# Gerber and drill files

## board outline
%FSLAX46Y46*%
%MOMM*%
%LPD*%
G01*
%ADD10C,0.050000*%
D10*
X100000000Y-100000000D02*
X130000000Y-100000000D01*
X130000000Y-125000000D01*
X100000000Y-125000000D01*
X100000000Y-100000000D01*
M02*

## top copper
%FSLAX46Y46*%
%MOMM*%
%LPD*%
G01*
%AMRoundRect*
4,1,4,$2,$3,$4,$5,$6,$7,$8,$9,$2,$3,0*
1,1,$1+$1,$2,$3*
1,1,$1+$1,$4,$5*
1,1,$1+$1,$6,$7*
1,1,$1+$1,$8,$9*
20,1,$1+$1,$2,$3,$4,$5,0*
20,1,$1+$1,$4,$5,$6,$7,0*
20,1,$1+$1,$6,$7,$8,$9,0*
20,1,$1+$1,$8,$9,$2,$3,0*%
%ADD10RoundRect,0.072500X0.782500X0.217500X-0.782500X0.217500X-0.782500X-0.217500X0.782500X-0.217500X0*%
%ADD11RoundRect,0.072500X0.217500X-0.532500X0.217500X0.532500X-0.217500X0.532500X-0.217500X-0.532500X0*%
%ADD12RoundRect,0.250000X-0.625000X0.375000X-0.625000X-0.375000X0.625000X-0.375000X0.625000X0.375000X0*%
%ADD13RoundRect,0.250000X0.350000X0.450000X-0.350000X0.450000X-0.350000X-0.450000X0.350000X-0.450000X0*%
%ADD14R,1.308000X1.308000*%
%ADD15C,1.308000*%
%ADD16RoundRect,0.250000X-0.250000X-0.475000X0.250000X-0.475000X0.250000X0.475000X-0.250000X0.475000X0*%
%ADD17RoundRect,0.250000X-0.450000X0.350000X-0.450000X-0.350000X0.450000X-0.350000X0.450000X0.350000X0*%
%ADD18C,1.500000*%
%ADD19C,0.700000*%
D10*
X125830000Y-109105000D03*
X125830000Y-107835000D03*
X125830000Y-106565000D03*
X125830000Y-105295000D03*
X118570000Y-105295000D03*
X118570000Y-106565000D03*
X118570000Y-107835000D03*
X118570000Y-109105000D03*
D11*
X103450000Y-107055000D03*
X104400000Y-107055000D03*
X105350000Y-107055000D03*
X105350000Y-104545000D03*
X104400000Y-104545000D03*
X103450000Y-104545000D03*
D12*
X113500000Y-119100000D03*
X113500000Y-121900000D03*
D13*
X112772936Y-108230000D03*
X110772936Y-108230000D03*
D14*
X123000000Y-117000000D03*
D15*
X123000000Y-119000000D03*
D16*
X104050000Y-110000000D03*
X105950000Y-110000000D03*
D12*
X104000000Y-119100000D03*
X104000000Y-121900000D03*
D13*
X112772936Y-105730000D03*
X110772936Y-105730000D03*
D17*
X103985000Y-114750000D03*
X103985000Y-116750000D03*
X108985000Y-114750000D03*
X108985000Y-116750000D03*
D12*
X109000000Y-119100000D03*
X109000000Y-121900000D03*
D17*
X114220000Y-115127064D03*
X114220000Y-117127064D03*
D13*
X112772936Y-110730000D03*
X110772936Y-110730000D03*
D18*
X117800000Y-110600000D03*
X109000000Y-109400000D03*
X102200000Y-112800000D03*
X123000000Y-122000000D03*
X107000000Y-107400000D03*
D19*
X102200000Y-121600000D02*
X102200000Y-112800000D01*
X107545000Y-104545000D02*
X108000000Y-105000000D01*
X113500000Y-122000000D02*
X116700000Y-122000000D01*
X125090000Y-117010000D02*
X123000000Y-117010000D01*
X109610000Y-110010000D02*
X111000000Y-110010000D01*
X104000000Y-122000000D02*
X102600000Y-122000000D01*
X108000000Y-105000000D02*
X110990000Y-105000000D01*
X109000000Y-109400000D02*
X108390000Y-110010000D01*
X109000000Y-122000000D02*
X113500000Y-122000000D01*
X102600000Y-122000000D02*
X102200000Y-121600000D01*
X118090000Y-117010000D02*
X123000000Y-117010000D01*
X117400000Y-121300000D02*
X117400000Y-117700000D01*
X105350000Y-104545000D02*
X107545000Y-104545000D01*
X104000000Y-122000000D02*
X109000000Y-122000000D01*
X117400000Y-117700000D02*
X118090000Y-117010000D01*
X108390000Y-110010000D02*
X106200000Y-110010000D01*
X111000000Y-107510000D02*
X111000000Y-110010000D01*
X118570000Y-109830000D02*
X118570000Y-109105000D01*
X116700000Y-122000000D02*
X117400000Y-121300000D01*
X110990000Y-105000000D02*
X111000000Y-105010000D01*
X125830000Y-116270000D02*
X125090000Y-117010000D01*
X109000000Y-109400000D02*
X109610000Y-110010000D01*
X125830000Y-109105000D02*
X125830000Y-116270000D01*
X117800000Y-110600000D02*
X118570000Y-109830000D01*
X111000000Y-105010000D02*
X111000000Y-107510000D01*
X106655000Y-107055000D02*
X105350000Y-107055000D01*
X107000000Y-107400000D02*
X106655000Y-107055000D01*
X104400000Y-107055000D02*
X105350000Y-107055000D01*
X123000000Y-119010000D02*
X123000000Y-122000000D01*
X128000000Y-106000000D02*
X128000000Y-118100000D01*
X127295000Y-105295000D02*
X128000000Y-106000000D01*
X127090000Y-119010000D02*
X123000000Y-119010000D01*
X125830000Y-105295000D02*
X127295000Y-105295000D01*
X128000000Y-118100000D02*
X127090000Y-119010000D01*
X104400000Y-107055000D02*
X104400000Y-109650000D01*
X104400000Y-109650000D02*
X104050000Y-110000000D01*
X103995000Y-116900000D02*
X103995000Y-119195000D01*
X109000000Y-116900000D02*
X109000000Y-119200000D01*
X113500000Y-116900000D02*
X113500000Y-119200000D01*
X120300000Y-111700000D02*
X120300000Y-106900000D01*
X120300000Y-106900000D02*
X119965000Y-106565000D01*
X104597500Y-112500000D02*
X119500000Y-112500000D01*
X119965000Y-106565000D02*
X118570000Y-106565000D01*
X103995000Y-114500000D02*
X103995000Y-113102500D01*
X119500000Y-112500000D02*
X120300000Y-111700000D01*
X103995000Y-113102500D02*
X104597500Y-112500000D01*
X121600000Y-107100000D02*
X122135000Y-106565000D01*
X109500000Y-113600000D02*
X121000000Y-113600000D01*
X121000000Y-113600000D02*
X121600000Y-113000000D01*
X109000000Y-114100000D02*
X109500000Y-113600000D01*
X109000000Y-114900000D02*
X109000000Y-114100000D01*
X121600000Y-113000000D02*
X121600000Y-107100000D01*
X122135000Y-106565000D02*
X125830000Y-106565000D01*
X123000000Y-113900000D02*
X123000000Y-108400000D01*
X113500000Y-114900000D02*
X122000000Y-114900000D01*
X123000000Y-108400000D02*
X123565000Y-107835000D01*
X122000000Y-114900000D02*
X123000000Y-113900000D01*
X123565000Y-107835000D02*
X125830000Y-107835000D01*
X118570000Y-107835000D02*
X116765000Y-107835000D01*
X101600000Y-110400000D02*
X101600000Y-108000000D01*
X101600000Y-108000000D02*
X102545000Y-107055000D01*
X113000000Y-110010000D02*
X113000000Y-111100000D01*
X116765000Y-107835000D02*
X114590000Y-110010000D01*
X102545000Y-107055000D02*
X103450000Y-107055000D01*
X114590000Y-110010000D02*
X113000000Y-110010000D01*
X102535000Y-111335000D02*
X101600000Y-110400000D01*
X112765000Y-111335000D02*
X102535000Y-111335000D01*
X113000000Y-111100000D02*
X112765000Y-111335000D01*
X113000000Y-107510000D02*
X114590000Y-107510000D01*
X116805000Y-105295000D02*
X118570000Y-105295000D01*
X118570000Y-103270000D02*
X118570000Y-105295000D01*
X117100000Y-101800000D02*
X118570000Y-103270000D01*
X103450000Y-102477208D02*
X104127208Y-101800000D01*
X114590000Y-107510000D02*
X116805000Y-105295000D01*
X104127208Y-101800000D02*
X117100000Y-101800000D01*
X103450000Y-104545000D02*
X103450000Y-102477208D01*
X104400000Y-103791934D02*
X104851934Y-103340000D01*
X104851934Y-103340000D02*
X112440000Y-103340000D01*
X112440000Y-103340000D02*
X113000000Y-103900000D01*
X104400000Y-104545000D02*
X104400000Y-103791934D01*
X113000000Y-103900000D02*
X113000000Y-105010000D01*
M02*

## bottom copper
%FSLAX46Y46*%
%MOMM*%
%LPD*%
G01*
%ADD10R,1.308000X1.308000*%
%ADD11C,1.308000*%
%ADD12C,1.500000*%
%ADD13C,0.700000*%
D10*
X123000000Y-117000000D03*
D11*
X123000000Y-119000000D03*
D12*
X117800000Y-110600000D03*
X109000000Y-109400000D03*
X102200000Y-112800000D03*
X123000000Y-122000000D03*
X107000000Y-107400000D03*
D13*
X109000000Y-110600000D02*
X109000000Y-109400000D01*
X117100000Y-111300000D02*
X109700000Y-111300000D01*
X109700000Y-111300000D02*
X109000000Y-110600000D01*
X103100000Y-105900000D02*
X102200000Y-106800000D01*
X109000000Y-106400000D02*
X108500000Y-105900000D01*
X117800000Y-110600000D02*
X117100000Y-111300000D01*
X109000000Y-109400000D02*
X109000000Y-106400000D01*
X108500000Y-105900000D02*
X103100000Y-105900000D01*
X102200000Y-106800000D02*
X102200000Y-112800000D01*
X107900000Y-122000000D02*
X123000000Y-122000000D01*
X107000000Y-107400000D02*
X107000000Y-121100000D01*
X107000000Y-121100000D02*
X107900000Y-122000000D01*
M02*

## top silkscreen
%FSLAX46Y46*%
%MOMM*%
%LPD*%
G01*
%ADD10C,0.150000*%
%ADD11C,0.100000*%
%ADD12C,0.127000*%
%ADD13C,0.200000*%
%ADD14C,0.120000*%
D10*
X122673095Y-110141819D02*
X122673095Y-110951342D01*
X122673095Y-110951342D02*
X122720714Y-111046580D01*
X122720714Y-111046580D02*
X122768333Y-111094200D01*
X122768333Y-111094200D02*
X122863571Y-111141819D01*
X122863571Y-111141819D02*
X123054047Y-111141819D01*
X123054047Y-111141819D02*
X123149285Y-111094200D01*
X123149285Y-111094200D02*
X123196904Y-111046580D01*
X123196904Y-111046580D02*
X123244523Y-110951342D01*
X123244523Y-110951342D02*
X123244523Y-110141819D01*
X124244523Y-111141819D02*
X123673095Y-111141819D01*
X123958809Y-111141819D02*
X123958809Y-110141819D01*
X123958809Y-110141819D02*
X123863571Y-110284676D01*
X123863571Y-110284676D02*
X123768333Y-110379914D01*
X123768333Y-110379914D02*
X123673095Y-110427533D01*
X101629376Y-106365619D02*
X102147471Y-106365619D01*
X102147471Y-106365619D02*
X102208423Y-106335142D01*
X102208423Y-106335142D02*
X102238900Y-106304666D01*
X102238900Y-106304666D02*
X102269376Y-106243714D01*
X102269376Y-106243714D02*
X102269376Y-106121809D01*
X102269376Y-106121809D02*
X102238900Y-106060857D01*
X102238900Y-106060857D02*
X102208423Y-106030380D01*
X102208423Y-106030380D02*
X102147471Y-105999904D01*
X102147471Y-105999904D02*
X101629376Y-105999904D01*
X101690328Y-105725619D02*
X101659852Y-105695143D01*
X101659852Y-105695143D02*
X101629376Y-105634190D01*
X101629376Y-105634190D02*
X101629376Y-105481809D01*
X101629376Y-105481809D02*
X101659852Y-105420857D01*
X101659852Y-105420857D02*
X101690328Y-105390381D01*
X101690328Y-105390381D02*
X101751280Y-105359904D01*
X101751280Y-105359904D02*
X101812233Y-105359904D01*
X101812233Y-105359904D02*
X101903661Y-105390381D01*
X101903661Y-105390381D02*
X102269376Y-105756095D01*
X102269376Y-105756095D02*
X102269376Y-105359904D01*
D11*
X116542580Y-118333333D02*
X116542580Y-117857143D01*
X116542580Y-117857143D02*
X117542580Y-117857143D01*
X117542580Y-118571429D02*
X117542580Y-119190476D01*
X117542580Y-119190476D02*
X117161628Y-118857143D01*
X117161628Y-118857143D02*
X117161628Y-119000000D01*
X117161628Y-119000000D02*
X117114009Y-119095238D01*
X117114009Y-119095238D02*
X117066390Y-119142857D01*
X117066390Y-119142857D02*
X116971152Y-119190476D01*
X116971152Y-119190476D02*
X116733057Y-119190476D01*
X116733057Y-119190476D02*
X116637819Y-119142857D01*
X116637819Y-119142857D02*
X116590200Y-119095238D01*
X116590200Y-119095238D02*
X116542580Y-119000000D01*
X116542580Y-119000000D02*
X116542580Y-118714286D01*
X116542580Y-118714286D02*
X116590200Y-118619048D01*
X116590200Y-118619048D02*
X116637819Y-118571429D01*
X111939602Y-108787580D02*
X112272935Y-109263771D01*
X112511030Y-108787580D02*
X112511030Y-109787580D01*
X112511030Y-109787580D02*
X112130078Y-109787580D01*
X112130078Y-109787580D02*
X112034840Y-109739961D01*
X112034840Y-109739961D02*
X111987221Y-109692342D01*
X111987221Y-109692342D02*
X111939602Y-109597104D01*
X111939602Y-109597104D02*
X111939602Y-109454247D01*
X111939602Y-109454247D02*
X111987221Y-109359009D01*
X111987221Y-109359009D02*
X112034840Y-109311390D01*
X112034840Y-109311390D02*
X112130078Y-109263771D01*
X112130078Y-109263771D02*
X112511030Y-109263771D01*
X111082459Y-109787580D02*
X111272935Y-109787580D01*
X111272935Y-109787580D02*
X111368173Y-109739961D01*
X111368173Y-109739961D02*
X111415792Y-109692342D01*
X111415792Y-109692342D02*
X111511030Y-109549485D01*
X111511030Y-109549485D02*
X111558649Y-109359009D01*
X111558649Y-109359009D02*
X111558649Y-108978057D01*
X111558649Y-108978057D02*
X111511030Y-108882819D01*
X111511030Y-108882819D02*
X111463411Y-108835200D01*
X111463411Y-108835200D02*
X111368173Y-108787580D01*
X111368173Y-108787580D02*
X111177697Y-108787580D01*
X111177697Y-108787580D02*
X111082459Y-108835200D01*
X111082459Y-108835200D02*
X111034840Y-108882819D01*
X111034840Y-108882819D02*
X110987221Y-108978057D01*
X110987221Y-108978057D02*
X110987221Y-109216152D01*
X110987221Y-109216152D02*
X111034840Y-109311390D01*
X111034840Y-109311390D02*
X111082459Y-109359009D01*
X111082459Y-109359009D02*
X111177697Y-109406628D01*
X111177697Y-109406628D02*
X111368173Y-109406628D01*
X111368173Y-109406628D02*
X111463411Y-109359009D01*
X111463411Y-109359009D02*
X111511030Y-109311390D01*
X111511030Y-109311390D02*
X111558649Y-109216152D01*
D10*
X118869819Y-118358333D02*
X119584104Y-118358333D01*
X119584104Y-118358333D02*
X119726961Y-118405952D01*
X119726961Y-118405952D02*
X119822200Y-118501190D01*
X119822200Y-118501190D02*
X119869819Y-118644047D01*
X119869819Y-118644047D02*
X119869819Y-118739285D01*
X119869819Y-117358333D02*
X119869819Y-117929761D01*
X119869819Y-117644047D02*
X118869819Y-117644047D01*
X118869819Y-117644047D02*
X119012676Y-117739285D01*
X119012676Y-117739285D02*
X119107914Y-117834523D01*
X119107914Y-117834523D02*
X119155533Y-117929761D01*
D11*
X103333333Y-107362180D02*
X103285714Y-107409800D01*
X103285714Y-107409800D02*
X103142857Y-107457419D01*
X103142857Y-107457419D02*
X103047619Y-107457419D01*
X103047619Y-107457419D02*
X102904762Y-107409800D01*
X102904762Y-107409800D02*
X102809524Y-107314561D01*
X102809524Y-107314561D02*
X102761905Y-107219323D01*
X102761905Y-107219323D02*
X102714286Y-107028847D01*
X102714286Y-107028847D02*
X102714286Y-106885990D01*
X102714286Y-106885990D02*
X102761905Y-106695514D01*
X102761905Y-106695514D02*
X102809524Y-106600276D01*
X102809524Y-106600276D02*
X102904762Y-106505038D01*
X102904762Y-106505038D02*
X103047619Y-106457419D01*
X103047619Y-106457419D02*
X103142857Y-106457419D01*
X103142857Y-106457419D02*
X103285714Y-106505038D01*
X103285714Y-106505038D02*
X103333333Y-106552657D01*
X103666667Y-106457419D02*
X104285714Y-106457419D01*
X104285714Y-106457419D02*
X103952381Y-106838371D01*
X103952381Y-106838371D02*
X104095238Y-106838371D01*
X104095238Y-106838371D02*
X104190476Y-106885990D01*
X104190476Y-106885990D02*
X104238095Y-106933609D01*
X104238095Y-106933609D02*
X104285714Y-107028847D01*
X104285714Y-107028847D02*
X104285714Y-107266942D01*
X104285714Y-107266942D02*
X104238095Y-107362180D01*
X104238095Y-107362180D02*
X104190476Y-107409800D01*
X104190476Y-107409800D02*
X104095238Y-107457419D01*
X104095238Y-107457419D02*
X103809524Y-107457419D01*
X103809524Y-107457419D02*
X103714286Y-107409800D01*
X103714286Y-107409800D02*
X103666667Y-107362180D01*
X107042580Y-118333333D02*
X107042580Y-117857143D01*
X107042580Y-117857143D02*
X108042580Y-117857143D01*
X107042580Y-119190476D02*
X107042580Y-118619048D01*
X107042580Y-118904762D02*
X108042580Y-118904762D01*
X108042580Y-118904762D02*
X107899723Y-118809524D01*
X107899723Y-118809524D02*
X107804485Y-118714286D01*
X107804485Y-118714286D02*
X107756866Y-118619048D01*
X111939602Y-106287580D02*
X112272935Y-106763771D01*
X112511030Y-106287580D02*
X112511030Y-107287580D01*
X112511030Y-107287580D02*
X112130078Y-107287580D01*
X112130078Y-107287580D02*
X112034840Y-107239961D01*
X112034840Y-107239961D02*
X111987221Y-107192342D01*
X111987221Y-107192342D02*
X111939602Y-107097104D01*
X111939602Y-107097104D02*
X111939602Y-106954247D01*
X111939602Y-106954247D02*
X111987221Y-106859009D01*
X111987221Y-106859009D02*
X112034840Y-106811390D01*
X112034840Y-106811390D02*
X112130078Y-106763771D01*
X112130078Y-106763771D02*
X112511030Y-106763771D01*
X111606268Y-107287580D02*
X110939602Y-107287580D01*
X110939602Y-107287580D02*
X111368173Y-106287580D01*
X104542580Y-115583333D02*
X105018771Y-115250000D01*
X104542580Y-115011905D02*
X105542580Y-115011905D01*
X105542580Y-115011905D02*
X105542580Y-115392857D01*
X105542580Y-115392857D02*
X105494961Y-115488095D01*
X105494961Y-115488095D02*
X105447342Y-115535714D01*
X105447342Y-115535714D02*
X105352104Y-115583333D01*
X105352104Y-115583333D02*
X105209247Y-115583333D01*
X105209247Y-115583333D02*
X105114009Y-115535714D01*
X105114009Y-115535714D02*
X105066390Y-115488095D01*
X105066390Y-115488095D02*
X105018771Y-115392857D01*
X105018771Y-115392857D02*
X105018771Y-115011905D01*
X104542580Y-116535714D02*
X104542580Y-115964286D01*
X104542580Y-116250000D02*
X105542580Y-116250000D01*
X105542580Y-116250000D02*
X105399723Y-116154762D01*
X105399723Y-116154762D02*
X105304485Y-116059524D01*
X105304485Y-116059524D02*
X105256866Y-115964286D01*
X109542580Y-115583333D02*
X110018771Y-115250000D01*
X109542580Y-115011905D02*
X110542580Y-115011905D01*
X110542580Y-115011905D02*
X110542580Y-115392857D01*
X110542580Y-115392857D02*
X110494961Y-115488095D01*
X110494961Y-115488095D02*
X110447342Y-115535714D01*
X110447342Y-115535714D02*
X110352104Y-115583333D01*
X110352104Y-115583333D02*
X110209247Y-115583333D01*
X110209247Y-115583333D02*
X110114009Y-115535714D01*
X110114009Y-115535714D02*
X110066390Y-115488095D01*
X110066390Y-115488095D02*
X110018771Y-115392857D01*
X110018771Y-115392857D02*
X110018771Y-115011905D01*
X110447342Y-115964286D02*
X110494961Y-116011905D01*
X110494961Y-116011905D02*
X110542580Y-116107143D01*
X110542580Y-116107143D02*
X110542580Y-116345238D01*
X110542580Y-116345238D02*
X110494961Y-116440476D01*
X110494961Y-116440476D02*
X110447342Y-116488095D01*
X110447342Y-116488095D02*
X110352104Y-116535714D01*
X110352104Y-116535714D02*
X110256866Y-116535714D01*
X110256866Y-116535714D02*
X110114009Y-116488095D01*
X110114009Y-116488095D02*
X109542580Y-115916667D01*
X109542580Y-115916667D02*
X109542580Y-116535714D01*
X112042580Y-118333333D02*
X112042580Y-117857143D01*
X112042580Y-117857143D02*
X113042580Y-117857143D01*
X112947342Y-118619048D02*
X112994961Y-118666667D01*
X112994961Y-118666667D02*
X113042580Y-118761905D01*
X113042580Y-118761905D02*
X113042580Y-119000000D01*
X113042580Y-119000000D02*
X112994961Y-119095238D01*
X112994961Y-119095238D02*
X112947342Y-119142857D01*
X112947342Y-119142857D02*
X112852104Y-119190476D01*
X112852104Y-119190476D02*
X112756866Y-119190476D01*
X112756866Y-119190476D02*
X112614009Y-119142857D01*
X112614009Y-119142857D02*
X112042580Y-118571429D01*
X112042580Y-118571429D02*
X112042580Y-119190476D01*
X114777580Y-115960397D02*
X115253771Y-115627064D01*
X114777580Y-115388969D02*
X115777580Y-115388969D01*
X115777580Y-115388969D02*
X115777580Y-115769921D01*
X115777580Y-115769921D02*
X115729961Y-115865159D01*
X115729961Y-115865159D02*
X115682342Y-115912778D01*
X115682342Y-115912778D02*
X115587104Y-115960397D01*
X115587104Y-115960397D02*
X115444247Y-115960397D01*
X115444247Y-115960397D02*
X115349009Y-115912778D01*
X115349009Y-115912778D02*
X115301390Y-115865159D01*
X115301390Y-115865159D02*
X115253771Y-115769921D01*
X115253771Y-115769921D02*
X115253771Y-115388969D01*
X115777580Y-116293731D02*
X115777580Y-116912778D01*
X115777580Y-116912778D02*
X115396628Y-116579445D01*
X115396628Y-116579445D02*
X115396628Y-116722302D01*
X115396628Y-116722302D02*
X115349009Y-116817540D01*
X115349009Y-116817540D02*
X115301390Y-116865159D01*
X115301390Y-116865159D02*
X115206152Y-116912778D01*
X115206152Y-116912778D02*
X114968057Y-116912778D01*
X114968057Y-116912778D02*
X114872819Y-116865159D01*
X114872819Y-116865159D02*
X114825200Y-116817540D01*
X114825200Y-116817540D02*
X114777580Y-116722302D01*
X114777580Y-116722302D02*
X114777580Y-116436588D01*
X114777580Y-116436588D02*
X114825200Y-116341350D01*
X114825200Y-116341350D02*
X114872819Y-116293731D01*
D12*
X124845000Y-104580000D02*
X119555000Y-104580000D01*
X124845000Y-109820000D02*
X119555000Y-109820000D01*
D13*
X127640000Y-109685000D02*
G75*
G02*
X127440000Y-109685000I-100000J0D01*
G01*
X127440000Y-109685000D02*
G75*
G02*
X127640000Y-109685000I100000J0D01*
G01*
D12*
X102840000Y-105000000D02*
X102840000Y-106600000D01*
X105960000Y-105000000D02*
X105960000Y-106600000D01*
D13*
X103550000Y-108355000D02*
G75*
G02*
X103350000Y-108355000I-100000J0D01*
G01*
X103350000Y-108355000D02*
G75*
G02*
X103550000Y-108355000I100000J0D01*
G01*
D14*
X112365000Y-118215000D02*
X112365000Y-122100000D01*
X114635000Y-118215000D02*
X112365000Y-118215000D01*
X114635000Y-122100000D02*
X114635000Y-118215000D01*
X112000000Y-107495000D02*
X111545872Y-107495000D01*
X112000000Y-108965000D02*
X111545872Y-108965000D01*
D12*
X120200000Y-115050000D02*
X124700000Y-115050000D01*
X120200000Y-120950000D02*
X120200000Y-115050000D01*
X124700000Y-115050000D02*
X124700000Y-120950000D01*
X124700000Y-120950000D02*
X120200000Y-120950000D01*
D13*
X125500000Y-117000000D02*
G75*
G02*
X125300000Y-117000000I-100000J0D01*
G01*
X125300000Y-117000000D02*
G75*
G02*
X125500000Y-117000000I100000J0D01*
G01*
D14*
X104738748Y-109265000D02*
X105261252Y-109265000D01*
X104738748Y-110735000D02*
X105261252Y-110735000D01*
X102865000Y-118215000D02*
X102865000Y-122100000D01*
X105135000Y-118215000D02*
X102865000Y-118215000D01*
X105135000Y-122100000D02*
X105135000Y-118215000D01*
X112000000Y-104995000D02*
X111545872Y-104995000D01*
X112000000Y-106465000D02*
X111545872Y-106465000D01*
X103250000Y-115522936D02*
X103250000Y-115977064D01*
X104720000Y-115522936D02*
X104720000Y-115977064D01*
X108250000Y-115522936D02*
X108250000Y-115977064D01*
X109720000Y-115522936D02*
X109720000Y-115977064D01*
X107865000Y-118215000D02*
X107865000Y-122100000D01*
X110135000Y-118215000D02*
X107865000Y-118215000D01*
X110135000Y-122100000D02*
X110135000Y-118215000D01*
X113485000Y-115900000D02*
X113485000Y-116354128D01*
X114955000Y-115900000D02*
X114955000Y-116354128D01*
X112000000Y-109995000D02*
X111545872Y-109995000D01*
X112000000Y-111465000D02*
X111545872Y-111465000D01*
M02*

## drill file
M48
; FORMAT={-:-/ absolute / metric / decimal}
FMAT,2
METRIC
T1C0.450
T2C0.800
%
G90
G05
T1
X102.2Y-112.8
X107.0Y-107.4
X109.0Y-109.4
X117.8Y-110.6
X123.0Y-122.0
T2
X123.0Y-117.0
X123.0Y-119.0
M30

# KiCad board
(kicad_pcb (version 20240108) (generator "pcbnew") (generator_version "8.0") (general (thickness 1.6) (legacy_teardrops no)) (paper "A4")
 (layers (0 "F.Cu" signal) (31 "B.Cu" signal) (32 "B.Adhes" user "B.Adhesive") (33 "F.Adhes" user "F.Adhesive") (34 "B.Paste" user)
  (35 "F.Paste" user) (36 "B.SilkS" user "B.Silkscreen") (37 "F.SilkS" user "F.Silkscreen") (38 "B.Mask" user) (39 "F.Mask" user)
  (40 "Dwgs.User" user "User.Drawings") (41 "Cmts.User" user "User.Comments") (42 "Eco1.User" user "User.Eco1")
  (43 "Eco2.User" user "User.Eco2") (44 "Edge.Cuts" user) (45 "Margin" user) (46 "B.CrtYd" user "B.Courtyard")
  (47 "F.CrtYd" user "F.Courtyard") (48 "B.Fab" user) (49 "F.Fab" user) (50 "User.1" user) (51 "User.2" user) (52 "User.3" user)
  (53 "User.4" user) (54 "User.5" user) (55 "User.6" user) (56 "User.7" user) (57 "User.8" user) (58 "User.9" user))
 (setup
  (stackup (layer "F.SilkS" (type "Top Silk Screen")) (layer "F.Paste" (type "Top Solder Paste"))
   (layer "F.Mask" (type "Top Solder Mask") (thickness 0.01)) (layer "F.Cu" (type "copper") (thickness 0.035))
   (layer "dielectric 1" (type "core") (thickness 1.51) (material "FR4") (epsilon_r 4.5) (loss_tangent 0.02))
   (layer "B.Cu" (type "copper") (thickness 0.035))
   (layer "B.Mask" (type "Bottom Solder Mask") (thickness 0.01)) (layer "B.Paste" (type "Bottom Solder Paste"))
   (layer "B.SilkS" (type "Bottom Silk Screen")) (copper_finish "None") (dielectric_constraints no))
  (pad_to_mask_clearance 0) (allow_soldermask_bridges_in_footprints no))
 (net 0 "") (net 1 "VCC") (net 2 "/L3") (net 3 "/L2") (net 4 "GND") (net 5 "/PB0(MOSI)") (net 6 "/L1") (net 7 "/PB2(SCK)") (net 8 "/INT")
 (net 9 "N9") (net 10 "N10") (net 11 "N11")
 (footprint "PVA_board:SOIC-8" (layer "F.Cu") (at 122.2 107.2 180)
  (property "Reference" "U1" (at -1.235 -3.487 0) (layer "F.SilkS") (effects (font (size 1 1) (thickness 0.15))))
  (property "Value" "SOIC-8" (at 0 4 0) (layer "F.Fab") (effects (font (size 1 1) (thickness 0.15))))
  (fp_line (start -2.645 2.62) (end 2.645 2.62) (stroke (width 0.127) (type solid)) (layer "F.SilkS"))
  (fp_line (start -2.645 -2.62) (end 2.645 -2.62) (stroke (width 0.127) (type solid)) (layer "F.SilkS"))
  (fp_circle (center -5.34 -2.485) (end -5.24 -2.485) (stroke (width 0.2) (type solid)) (fill none) (layer "F.SilkS"))
  (pad "1" smd roundrect (at -3.63 -1.905 180) (size 1.71 0.58) (layers "F.Cu" "F.Paste" "F.Mask") (roundrect_rratio 0.125) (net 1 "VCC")
   (solder_mask_margin 0.102))
  (pad "2" smd roundrect (at -3.63 -0.635 180) (size 1.71 0.58) (layers "F.Cu" "F.Paste" "F.Mask") (roundrect_rratio 0.125) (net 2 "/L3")
   (solder_mask_margin 0.102))
  (pad "3" smd roundrect (at -3.63 0.635 180) (size 1.71 0.58) (layers "F.Cu" "F.Paste" "F.Mask") (roundrect_rratio 0.125) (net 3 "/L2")
   (solder_mask_margin 0.102))
  (pad "4" smd roundrect (at -3.63 1.905 180) (size 1.71 0.58) (layers "F.Cu" "F.Paste" "F.Mask") (roundrect_rratio 0.125) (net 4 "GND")
   (solder_mask_margin 0.102))
  (pad "5" smd roundrect (at 3.63 1.905 180) (size 1.71 0.58) (layers "F.Cu" "F.Paste" "F.Mask") (roundrect_rratio 0.125)
   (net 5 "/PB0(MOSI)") (solder_mask_margin 0.102))
  (pad "6" smd roundrect (at 3.63 0.635 180) (size 1.71 0.58) (layers "F.Cu" "F.Paste" "F.Mask") (roundrect_rratio 0.125) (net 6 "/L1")
   (solder_mask_margin 0.102))
  (pad "7" smd roundrect (at 3.63 -0.635 180) (size 1.71 0.58) (layers "F.Cu" "F.Paste" "F.Mask") (roundrect_rratio 0.125)
   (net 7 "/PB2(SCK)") (solder_mask_margin 0.102))
  (pad "8" smd roundrect (at 3.63 -1.905 180) (size 1.71 0.58) (layers "F.Cu" "F.Paste" "F.Mask") (roundrect_rratio 0.125) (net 1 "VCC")
   (solder_mask_margin 0.102)))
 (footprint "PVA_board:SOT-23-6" (layer "F.Cu") (at 104.4 105.8 90)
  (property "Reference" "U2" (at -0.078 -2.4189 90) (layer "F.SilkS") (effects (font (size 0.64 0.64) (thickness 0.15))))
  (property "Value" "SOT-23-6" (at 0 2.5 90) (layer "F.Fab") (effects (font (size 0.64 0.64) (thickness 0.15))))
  (fp_line (start 0.8 -1.56) (end -0.8 -1.56) (stroke (width 0.127) (type solid)) (layer "F.SilkS"))
  (fp_line (start 0.8 1.56) (end -0.8 1.56) (stroke (width 0.127) (type solid)) (layer "F.SilkS"))
  (fp_circle (center -2.555 -0.95) (end -2.455 -0.95) (stroke (width 0.2) (type solid)) (fill none) (layer "F.SilkS"))
  (pad "1" smd roundrect (at -1.255 -0.95 90) (size 1.21 0.58) (layers "F.Cu" "F.Paste" "F.Mask") (roundrect_rratio 0.125)
   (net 7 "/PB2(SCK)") (solder_mask_margin 0.102))
  (pad "2" smd roundrect (at -1.255 0 90) (size 1.21 0.58) (layers "F.Cu" "F.Paste" "F.Mask") (roundrect_rratio 0.125) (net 4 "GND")
   (solder_mask_margin 0.102))
  (pad "3" smd roundrect (at -1.255 0.95 90) (size 1.21 0.58) (layers "F.Cu" "F.Paste" "F.Mask") (roundrect_rratio 0.125) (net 4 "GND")
   (solder_mask_margin 0.102))
  (pad "4" smd roundrect (at 1.255 0.95 90) (size 1.21 0.58) (layers "F.Cu" "F.Paste" "F.Mask") (roundrect_rratio 0.125) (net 1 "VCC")
   (solder_mask_margin 0.102))
  (pad "5" smd roundrect (at 1.255 0 90) (size 1.21 0.58) (layers "F.Cu" "F.Paste" "F.Mask") (roundrect_rratio 0.125) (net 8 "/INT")
   (solder_mask_margin 0.102))
  (pad "6" smd roundrect (at 1.255 -0.95 90) (size 1.21 0.58) (layers "F.Cu" "F.Paste" "F.Mask") (roundrect_rratio 0.125)
   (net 5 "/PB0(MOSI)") (solder_mask_margin 0.102)))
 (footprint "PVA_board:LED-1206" (layer "F.Cu") (at 113.5 120.5 -90)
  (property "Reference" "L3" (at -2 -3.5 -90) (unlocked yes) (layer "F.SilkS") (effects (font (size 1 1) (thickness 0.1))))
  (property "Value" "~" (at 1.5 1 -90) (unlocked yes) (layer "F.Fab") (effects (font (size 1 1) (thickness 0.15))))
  (fp_line (start -2.285 1.135) (end 1.6 1.135) (stroke (width 0.12) (type solid)) (layer "F.SilkS"))
  (fp_line (start -2.285 -1.135) (end -2.285 1.135) (stroke (width 0.12) (type solid)) (layer "F.SilkS"))
  (fp_line (start 1.6 -1.135) (end -2.285 -1.135) (stroke (width 0.12) (type solid)) (layer "F.SilkS"))
  (pad "1" smd roundrect (at -1.4 0 270) (size 1.25 1.75) (layers "F.Cu" "F.Paste" "F.Mask") (roundrect_rratio 0.2) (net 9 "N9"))
  (pad "2" smd roundrect (at 1.4 0 270) (size 1.25 1.75) (layers "F.Cu" "F.Paste" "F.Mask") (roundrect_rratio 0.2) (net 1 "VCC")))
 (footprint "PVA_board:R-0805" (layer "F.Cu") (at 111.772936 108.245 180)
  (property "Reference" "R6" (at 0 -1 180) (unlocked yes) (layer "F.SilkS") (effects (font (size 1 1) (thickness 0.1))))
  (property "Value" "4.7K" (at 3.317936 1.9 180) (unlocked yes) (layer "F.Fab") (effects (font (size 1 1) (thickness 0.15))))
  (fp_line (start -0.227064 0.75) (end 0.227064 0.75) (stroke (width 0.12) (type solid)) (layer "F.SilkS"))
  (fp_line (start -0.227064 -0.72) (end 0.227064 -0.72) (stroke (width 0.12) (type solid)) (layer "F.SilkS"))
  (pad "1" smd roundrect (at -1 0.015 180) (size 1.2 1.4) (layers "F.Cu" "F.Paste" "F.Mask") (roundrect_rratio 0.208333)
   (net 5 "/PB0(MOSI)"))
  (pad "2" smd roundrect (at 1 0.015 180) (size 1.2 1.4) (layers "F.Cu" "F.Paste" "F.Mask") (roundrect_rratio 0.208333) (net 1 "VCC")))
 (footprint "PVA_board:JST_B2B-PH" (layer "F.Cu") (at 123 118 90)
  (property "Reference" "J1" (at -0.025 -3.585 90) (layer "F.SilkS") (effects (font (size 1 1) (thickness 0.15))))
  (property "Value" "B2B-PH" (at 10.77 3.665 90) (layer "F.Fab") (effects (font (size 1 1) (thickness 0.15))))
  (fp_line (start 2.95 -2.8) (end 2.95 1.7) (stroke (width 0.127) (type solid)) (layer "F.SilkS"))
  (fp_line (start -2.95 -2.8) (end 2.95 -2.8) (stroke (width 0.127) (type solid)) (layer "F.SilkS"))
  (fp_line (start 2.95 1.7) (end -2.95 1.7) (stroke (width 0.127) (type solid)) (layer "F.SilkS"))
  (fp_line (start -2.95 1.7) (end -2.95 -2.8) (stroke (width 0.127) (type solid)) (layer "F.SilkS"))
  (fp_circle (center 1 2.4) (end 1.1 2.4) (stroke (width 0.2) (type solid)) (fill none) (layer "F.SilkS"))
  (pad "1" thru_hole rect (at 1 0 90) (size 1.308 1.308) (drill 0.8) (layers "*.Cu" "*.Mask") (remove_unused_layers no) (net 1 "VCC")
   (solder_mask_margin 0.102))
  (pad "2" thru_hole circle (at -1 0 90) (size 1.308 1.308) (drill 0.8) (layers "*.Cu" "*.Mask") (remove_unused_layers no) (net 4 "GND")
   (solder_mask_margin 0.102)))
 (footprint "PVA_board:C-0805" (layer "F.Cu") (at 105 110)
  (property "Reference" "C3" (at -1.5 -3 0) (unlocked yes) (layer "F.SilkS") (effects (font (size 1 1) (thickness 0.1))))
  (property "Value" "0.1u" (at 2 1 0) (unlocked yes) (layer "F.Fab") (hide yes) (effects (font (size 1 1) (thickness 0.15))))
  (fp_line (start -0.261252 -0.735) (end 0.261252 -0.735) (stroke (width 0.12) (type solid)) (layer "F.SilkS"))
  (fp_line (start -0.261252 0.735) (end 0.261252 0.735) (stroke (width 0.12) (type solid)) (layer "F.SilkS"))
  (pad "1" smd roundrect (at -0.95 0) (size 1 1.45) (layers "F.Cu" "F.Paste" "F.Mask") (roundrect_rratio 0.25) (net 4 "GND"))
  (pad "2" smd roundrect (at 0.95 0) (size 1 1.45) (layers "F.Cu" "F.Paste" "F.Mask") (roundrect_rratio 0.25) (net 1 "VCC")))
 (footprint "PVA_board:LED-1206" (layer "F.Cu") (at 104 120.5 -90)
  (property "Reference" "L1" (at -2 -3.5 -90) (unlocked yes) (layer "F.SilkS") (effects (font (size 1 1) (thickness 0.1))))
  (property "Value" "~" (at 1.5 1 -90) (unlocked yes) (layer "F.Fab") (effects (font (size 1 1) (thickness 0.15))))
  (fp_line (start -2.285 1.135) (end 1.6 1.135) (stroke (width 0.12) (type solid)) (layer "F.SilkS"))
  (fp_line (start -2.285 -1.135) (end -2.285 1.135) (stroke (width 0.12) (type solid)) (layer "F.SilkS"))
  (fp_line (start 1.6 -1.135) (end -2.285 -1.135) (stroke (width 0.12) (type solid)) (layer "F.SilkS"))
  (pad "1" smd roundrect (at -1.4 0 270) (size 1.25 1.75) (layers "F.Cu" "F.Paste" "F.Mask") (roundrect_rratio 0.2) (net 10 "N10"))
  (pad "2" smd roundrect (at 1.4 0 270) (size 1.25 1.75) (layers "F.Cu" "F.Paste" "F.Mask") (roundrect_rratio 0.2) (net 1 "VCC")))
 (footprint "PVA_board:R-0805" (layer "F.Cu") (at 111.772936 105.745 180)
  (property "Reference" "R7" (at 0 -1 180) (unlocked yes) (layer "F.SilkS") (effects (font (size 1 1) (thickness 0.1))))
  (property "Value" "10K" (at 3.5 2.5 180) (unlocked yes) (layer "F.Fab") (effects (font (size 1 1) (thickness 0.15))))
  (fp_line (start -0.227064 0.75) (end 0.227064 0.75) (stroke (width 0.12) (type solid)) (layer "F.SilkS"))
  (fp_line (start -0.227064 -0.72) (end 0.227064 -0.72) (stroke (width 0.12) (type solid)) (layer "F.SilkS"))
  (pad "1" smd roundrect (at -1 0.015 180) (size 1.2 1.4) (layers "F.Cu" "F.Paste" "F.Mask") (roundrect_rratio 0.208333) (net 8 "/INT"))
  (pad "2" smd roundrect (at 1 0.015 180) (size 1.2 1.4) (layers "F.Cu" "F.Paste" "F.Mask") (roundrect_rratio 0.208333) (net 1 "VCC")))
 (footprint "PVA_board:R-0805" (layer "F.Cu") (at 104 115.75 -90)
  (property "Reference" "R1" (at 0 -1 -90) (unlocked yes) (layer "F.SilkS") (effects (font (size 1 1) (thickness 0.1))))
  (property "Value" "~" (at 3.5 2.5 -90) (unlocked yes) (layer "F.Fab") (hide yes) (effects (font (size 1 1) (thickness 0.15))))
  (fp_line (start -0.227064 0.75) (end 0.227064 0.75) (stroke (width 0.12) (type solid)) (layer "F.SilkS"))
  (fp_line (start -0.227064 -0.72) (end 0.227064 -0.72) (stroke (width 0.12) (type solid)) (layer "F.SilkS"))
  (pad "1" smd roundrect (at -1 0.015 270) (size 1.2 1.4) (layers "F.Cu" "F.Paste" "F.Mask") (roundrect_rratio 0.208333) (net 6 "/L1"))
  (pad "2" smd roundrect (at 1 0.015 270) (size 1.2 1.4) (layers "F.Cu" "F.Paste" "F.Mask") (roundrect_rratio 0.208333) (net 10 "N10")))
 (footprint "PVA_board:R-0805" (layer "F.Cu") (at 109 115.75 -90)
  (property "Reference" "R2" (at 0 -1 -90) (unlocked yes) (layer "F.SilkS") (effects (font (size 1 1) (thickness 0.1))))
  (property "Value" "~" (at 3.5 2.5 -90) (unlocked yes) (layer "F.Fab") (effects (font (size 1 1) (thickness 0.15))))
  (fp_line (start -0.227064 0.75) (end 0.227064 0.75) (stroke (width 0.12) (type solid)) (layer "F.SilkS"))
  (fp_line (start -0.227064 -0.72) (end 0.227064 -0.72) (stroke (width 0.12) (type solid)) (layer "F.SilkS"))
  (pad "1" smd roundrect (at -1 0.015 270) (size 1.2 1.4) (layers "F.Cu" "F.Paste" "F.Mask") (roundrect_rratio 0.208333) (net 3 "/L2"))
  (pad "2" smd roundrect (at 1 0.015 270) (size 1.2 1.4) (layers "F.Cu" "F.Paste" "F.Mask") (roundrect_rratio 0.208333) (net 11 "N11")))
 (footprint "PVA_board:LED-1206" (layer "F.Cu") (at 109 120.5 -90)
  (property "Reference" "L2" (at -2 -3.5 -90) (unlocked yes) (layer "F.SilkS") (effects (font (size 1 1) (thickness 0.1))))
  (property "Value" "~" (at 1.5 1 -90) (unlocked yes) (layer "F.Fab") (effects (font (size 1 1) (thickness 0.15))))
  (fp_line (start -2.285 1.135) (end 1.6 1.135) (stroke (width 0.12) (type solid)) (layer "F.SilkS"))
  (fp_line (start -2.285 -1.135) (end -2.285 1.135) (stroke (width 0.12) (type solid)) (layer "F.SilkS"))
  (fp_line (start 1.6 -1.135) (end -2.285 -1.135) (stroke (width 0.12) (type solid)) (layer "F.SilkS"))
  (pad "1" smd roundrect (at -1.4 0 270) (size 1.25 1.75) (layers "F.Cu" "F.Paste" "F.Mask") (roundrect_rratio 0.2) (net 11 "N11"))
  (pad "2" smd roundrect (at 1.4 0 270) (size 1.25 1.75) (layers "F.Cu" "F.Paste" "F.Mask") (roundrect_rratio 0.2) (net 1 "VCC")))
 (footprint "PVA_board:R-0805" (layer "F.Cu") (at 114.235 116.127064 -90)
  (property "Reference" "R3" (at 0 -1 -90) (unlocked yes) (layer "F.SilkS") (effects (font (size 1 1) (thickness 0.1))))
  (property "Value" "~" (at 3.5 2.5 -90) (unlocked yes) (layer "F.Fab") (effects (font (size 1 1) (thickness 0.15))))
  (fp_line (start -0.227064 0.75) (end 0.227064 0.75) (stroke (width 0.12) (type solid)) (layer "F.SilkS"))
  (fp_line (start -0.227064 -0.72) (end 0.227064 -0.72) (stroke (width 0.12) (type solid)) (layer "F.SilkS"))
  (pad "1" smd roundrect (at -1 0.015 270) (size 1.2 1.4) (layers "F.Cu" "F.Paste" "F.Mask") (roundrect_rratio 0.208333) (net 2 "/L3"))
  (pad "2" smd roundrect (at 1 0.015 270) (size 1.2 1.4) (layers "F.Cu" "F.Paste" "F.Mask") (roundrect_rratio 0.208333) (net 9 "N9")))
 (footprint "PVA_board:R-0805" (layer "F.Cu") (at 111.772936 110.745 180)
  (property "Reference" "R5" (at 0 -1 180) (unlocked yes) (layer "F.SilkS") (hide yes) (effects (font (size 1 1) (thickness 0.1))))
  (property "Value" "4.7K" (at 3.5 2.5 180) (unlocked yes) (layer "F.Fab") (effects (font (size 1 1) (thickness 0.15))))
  (fp_line (start -0.227064 0.75) (end 0.227064 0.75) (stroke (width 0.12) (type solid)) (layer "F.SilkS"))
  (fp_line (start -0.227064 -0.72) (end 0.227064 -0.72) (stroke (width 0.12) (type solid)) (layer "F.SilkS"))
  (pad "1" smd roundrect (at -1 0.015 180) (size 1.2 1.4) (layers "F.Cu" "F.Paste" "F.Mask") (roundrect_rratio 0.208333) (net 7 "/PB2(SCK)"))
  (pad "2" smd roundrect (at 1 0.015 180) (size 1.2 1.4) (layers "F.Cu" "F.Paste" "F.Mask") (roundrect_rratio 0.208333) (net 1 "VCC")))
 (gr_rect (start 100 100) (end 130 125) (stroke (width 0.05) (type default)) (fill none) (layer "Edge.Cuts"))
 (segment (start 102.2 121.6) (end 102.2 112.8) (width 0.7) (layer "F.Cu") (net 1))
 (segment (start 107.545 104.545) (end 108 105) (width 0.7) (layer "F.Cu") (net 1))
 (segment (start 113.5 122) (end 116.7 122) (width 0.7) (layer "F.Cu") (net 1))
 (segment (start 125.09 117.01) (end 123 117.01) (width 0.7) (layer "F.Cu") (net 1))
 (segment (start 109.61 110.01) (end 111 110.01) (width 0.7) (layer "F.Cu") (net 1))
 (segment (start 104 122) (end 102.6 122) (width 0.7) (layer "F.Cu") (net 1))
 (segment (start 108 105) (end 110.99 105) (width 0.7) (layer "F.Cu") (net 1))
 (segment (start 109 109.4) (end 108.39 110.01) (width 0.7) (layer "F.Cu") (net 1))
 (segment (start 109 122) (end 113.5 122) (width 0.7) (layer "F.Cu") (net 1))
 (segment (start 102.6 122) (end 102.2 121.6) (width 0.7) (layer "F.Cu") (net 1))
 (segment (start 118.09 117.01) (end 123 117.01) (width 0.7) (layer "F.Cu") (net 1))
 (segment (start 117.4 121.3) (end 117.4 117.7) (width 0.7) (layer "F.Cu") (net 1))
 (segment (start 105.35 104.545) (end 107.545 104.545) (width 0.7) (layer "F.Cu") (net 1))
 (segment (start 104 122) (end 109 122) (width 0.7) (layer "F.Cu") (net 1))
 (segment (start 117.4 117.7) (end 118.09 117.01) (width 0.7) (layer "F.Cu") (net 1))
 (segment (start 108.39 110.01) (end 106.2 110.01) (width 0.7) (layer "F.Cu") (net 1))
 (segment (start 111 107.51) (end 111 110.01) (width 0.7) (layer "F.Cu") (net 1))
 (segment (start 118.57 109.83) (end 118.57 109.105) (width 0.7) (layer "F.Cu") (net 1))
 (segment (start 116.7 122) (end 117.4 121.3) (width 0.7) (layer "F.Cu") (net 1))
 (segment (start 110.99 105) (end 111 105.01) (width 0.7) (layer "F.Cu") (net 1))
 (segment (start 125.83 116.27) (end 125.09 117.01) (width 0.7) (layer "F.Cu") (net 1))
 (segment (start 109 109.4) (end 109.61 110.01) (width 0.7) (layer "F.Cu") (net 1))
 (segment (start 125.83 109.105) (end 125.83 116.27) (width 0.7) (layer "F.Cu") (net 1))
 (segment (start 117.8 110.6) (end 118.57 109.83) (width 0.7) (layer "F.Cu") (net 1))
 (segment (start 111 105.01) (end 111 107.51) (width 0.7) (layer "F.Cu") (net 1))
 (via (at 117.8 110.6) (size 1.5) (drill 0.45) (layers "F.Cu" "B.Cu") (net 1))
 (via (at 109 109.4) (size 1.5) (drill 0.45) (layers "F.Cu" "B.Cu") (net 1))
 (via (at 102.2 112.8) (size 1.5) (drill 0.45) (layers "F.Cu" "B.Cu") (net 1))
 (segment (start 109 110.6) (end 109 109.4) (width 0.7) (layer "B.Cu") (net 1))
 (segment (start 117.1 111.3) (end 109.7 111.3) (width 0.7) (layer "B.Cu") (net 1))
 (segment (start 109.7 111.3) (end 109 110.6) (width 0.7) (layer "B.Cu") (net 1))
 (segment (start 103.1 105.9) (end 102.2 106.8) (width 0.7) (layer "B.Cu") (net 1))
 (segment (start 109 106.4) (end 108.5 105.9) (width 0.7) (layer "B.Cu") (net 1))
 (segment (start 117.8 110.6) (end 117.1 111.3) (width 0.7) (layer "B.Cu") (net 1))
 (segment (start 109 109.4) (end 109 106.4) (width 0.7) (layer "B.Cu") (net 1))
 (segment (start 108.5 105.9) (end 103.1 105.9) (width 0.7) (layer "B.Cu") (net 1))
 (segment (start 102.2 106.8) (end 102.2 112.8) (width 0.7) (layer "B.Cu") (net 1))
 (segment (start 106.655 107.055) (end 105.35 107.055) (width 0.7) (layer "F.Cu") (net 4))
 (segment (start 107 107.4) (end 106.655 107.055) (width 0.7) (layer "F.Cu") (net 4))
 (segment (start 104.4 107.055) (end 105.35 107.055) (width 0.7) (layer "F.Cu") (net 4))
 (segment (start 123 119.01) (end 123 122) (width 0.7) (layer "F.Cu") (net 4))
 (segment (start 128 106) (end 128 118.1) (width 0.7) (layer "F.Cu") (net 4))
 (segment (start 127.295 105.295) (end 128 106) (width 0.7) (layer "F.Cu") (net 4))
 (segment (start 127.09 119.01) (end 123 119.01) (width 0.7) (layer "F.Cu") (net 4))
 (segment (start 125.83 105.295) (end 127.295 105.295) (width 0.7) (layer "F.Cu") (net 4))
 (segment (start 128 118.1) (end 127.09 119.01) (width 0.7) (layer "F.Cu") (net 4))
 (segment (start 104.4 107.055) (end 104.4 109.65) (width 0.7) (layer "F.Cu") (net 4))
 (segment (start 104.4 109.65) (end 104.05 110) (width 0.7) (layer "F.Cu") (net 4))
 (via (at 123 122) (size 1.5) (drill 0.45) (layers "F.Cu" "B.Cu") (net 4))
 (via (at 107 107.4) (size 1.5) (drill 0.45) (layers "F.Cu" "B.Cu") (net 4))
 (segment (start 107.9 122) (end 123 122) (width 0.7) (layer "B.Cu") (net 4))
 (segment (start 107 107.4) (end 107 121.1) (width 0.7) (layer "B.Cu") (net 4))
 (segment (start 107 121.1) (end 107.9 122) (width 0.7) (layer "B.Cu") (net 4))
 (segment (start 103.995 116.9) (end 103.995 119.195) (width 0.7) (layer "F.Cu") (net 10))
 (segment (start 109 116.9) (end 109 119.2) (width 0.7) (layer "F.Cu") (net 11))
 (segment (start 113.5 116.9) (end 113.5 119.2) (width 0.7) (layer "F.Cu") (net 9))
 (segment (start 120.3 111.7) (end 120.3 106.9) (width 0.7) (layer "F.Cu") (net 6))
 (segment (start 120.3 106.9) (end 119.965 106.565) (width 0.7) (layer "F.Cu") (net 6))
 (segment (start 104.5975 112.5) (end 119.5 112.5) (width 0.7) (layer "F.Cu") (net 6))
 (segment (start 119.965 106.565) (end 118.57 106.565) (width 0.7) (layer "F.Cu") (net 6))
 (segment (start 103.995 114.5) (end 103.995 113.1025) (width 0.7) (layer "F.Cu") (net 6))
 (segment (start 119.5 112.5) (end 120.3 111.7) (width 0.7) (layer "F.Cu") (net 6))
 (segment (start 103.995 113.1025) (end 104.5975 112.5) (width 0.7) (layer "F.Cu") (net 6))
 (segment (start 121.6 107.1) (end 122.135 106.565) (width 0.7) (layer "F.Cu") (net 3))
 (segment (start 109.5 113.6) (end 121 113.6) (width 0.7) (layer "F.Cu") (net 3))
 (segment (start 121 113.6) (end 121.6 113) (width 0.7) (layer "F.Cu") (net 3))
 (segment (start 109 114.1) (end 109.5 113.6) (width 0.7) (layer "F.Cu") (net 3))
 (segment (start 109 114.9) (end 109 114.1) (width 0.7) (layer "F.Cu") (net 3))
 (segment (start 121.6 113) (end 121.6 107.1) (width 0.7) (layer "F.Cu") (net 3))
 (segment (start 122.135 106.565) (end 125.83 106.565) (width 0.7) (layer "F.Cu") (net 3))
 (segment (start 123 113.9) (end 123 108.4) (width 0.7) (layer "F.Cu") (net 2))
 (segment (start 113.5 114.9) (end 122 114.9) (width 0.7) (layer "F.Cu") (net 2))
 (segment (start 123 108.4) (end 123.565 107.835) (width 0.7) (layer "F.Cu") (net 2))
 (segment (start 122 114.9) (end 123 113.9) (width 0.7) (layer "F.Cu") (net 2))
 (segment (start 123.565 107.835) (end 125.83 107.835) (width 0.7) (layer "F.Cu") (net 2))
 (segment (start 118.57 107.835) (end 116.765 107.835) (width 0.7) (layer "F.Cu") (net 7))
 (segment (start 101.6 110.4) (end 101.6 108) (width 0.7) (layer "F.Cu") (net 7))
 (segment (start 101.6 108) (end 102.545 107.055) (width 0.7) (layer "F.Cu") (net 7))
 (segment (start 113 110.01) (end 113 111.1) (width 0.7) (layer "F.Cu") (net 7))
 (segment (start 116.765 107.835) (end 114.59 110.01) (width 0.7) (layer "F.Cu") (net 7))
 (segment (start 102.545 107.055) (end 103.45 107.055) (width 0.7) (layer "F.Cu") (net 7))
 (segment (start 114.59 110.01) (end 113 110.01) (width 0.7) (layer "F.Cu") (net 7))
 (segment (start 102.535 111.335) (end 101.6 110.4) (width 0.7) (layer "F.Cu") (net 7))
 (segment (start 112.765 111.335) (end 102.535 111.335) (width 0.7) (layer "F.Cu") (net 7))
 (segment (start 113 111.1) (end 112.765 111.335) (width 0.7) (layer "F.Cu") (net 7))
 (segment (start 113 107.51) (end 114.59 107.51) (width 0.7) (layer "F.Cu") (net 5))
 (segment (start 116.805 105.295) (end 118.57 105.295) (width 0.7) (layer "F.Cu") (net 5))
 (segment (start 118.57 103.27) (end 118.57 105.295) (width 0.7) (layer "F.Cu") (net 5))
 (segment (start 117.1 101.8) (end 118.57 103.27) (width 0.7) (layer "F.Cu") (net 5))
 (segment (start 103.45 102.477208) (end 104.127208 101.8) (width 0.7) (layer "F.Cu") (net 5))
 (segment (start 114.59 107.51) (end 116.805 105.295) (width 0.7) (layer "F.Cu") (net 5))
 (segment (start 104.127208 101.8) (end 117.1 101.8) (width 0.7) (layer "F.Cu") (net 5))
 (segment (start 103.45 104.545) (end 103.45 102.477208) (width 0.7) (layer "F.Cu") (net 5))
 (segment (start 104.4 103.791934) (end 104.851934 103.34) (width 0.7) (layer "F.Cu") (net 8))
 (segment (start 104.851934 103.34) (end 112.44 103.34) (width 0.7) (layer "F.Cu") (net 8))
 (segment (start 112.44 103.34) (end 113 103.9) (width 0.7) (layer "F.Cu") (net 8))
 (segment (start 104.4 104.545) (end 104.4 103.791934) (width 0.7) (layer "F.Cu") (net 8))
 (segment (start 113 103.9) (end 113 105.01) (width 0.7) (layer "F.Cu") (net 8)))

